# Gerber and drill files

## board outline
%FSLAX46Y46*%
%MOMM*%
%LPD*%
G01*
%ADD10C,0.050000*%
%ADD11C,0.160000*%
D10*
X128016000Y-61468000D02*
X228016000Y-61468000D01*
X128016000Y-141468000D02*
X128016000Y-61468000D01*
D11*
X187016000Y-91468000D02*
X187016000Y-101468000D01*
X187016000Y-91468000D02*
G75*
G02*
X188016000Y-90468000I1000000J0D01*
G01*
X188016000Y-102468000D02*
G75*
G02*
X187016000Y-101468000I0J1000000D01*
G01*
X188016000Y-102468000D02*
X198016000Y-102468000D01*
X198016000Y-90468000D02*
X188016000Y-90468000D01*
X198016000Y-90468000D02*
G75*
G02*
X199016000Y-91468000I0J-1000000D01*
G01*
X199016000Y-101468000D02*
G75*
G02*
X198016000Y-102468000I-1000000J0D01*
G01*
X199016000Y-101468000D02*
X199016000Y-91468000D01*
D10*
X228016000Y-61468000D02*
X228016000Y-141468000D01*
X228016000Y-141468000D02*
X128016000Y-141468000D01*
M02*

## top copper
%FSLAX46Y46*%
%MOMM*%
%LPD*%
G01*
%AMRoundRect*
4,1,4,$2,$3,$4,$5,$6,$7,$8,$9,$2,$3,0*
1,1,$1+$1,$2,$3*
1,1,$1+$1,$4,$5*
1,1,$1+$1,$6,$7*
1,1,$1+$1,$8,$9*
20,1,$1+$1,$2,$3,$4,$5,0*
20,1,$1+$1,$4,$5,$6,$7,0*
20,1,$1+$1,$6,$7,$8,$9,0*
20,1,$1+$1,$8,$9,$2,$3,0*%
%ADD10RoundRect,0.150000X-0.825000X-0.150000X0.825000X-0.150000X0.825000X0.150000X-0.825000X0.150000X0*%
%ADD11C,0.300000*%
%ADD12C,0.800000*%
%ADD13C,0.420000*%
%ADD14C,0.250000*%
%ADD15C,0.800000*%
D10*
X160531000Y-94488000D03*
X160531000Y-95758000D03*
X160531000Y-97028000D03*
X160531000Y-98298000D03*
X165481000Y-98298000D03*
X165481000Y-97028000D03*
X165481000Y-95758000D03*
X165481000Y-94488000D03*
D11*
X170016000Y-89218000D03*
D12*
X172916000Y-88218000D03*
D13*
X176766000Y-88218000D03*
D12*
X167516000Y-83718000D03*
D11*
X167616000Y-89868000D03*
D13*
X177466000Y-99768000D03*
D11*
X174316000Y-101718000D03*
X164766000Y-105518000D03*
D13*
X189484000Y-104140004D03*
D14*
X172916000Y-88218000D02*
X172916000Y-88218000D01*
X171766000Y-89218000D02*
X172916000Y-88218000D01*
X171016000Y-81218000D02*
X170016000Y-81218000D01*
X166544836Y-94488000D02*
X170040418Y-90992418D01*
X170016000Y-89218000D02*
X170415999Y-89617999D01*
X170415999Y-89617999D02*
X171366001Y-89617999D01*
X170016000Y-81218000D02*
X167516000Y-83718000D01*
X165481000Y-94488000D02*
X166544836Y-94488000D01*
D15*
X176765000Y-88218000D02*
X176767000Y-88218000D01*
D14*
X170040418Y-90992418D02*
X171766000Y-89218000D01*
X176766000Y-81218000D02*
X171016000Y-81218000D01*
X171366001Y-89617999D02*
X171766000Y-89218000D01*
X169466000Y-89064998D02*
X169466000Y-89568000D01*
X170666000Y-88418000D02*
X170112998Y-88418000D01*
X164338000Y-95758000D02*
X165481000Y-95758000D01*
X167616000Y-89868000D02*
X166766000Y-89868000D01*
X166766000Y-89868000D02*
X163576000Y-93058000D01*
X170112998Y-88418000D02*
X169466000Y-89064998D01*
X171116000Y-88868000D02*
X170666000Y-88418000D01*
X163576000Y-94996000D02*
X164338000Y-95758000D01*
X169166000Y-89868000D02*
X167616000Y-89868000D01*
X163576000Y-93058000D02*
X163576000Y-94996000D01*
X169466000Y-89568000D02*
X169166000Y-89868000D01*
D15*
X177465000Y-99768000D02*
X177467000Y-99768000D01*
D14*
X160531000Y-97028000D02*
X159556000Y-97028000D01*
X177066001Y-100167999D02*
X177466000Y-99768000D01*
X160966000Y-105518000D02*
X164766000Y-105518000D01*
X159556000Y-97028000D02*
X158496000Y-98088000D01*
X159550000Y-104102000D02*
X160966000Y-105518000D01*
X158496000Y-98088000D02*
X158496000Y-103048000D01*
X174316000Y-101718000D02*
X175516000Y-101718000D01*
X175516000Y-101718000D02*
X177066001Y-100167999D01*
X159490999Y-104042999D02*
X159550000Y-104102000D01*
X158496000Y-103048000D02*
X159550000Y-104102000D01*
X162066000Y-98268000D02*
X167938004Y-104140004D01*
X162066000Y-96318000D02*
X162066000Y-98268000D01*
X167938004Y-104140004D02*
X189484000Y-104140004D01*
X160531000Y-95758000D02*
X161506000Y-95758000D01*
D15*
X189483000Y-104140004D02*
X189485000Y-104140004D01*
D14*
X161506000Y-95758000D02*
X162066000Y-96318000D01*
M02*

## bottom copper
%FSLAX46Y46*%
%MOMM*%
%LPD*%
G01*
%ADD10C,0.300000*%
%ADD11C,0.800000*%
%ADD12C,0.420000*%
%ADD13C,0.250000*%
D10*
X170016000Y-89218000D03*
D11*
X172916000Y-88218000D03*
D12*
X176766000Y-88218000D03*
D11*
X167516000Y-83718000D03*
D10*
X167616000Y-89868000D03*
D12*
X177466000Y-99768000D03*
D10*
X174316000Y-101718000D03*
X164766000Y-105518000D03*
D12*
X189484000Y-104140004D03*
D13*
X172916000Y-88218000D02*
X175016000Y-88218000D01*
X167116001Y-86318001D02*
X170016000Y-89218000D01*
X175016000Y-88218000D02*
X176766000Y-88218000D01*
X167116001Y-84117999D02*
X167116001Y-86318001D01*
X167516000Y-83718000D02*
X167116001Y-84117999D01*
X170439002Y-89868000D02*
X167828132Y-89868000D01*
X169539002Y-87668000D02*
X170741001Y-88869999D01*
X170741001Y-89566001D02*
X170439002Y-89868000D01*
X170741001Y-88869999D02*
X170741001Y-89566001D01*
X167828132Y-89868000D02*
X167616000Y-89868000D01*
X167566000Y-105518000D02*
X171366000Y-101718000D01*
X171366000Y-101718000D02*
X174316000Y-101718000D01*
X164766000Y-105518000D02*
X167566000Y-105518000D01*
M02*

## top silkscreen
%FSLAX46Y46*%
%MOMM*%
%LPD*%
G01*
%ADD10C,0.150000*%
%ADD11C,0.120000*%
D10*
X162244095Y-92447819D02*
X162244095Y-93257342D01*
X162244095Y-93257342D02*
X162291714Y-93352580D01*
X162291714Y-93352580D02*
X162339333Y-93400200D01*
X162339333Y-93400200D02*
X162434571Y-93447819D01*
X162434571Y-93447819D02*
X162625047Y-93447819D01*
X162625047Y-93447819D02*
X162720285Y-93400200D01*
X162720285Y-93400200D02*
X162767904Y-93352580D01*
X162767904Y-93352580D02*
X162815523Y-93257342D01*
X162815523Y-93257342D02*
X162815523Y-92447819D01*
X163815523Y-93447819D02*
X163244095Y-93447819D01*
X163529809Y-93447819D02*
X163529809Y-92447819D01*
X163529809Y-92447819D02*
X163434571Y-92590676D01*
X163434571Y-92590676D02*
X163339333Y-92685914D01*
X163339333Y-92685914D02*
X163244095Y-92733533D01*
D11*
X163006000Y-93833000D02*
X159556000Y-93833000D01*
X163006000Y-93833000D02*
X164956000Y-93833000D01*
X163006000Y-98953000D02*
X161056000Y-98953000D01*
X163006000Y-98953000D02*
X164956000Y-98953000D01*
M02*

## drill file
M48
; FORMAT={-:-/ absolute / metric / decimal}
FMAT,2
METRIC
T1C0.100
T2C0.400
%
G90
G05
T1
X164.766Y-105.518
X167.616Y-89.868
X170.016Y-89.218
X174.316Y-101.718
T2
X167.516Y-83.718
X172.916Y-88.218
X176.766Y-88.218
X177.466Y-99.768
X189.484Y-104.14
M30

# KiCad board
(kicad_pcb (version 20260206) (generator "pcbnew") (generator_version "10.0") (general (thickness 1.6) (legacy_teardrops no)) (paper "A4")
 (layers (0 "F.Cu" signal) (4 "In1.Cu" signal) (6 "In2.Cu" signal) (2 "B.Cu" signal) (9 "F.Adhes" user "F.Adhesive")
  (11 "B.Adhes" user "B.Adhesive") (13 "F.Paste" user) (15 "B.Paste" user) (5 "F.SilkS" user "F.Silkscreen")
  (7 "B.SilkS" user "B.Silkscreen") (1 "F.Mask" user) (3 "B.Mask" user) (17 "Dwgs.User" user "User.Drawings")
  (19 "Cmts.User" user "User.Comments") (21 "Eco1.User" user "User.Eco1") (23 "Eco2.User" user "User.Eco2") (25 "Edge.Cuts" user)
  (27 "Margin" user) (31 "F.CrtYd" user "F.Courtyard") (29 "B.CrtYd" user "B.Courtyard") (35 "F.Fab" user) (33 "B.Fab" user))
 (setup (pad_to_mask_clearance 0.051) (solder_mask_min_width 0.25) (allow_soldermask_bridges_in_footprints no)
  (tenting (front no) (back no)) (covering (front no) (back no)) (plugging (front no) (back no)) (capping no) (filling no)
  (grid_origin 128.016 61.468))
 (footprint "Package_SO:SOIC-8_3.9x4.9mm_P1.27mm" (layer "F.Cu") (at 163.006 96.393)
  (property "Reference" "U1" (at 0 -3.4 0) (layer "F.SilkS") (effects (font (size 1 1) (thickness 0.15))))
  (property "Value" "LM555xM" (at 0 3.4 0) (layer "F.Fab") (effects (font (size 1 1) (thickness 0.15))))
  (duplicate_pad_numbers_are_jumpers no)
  (fp_line (start 0 -2.56) (end -3.45 -2.56) (stroke (width 0.12) (type solid)) (layer "F.SilkS"))
  (fp_line (start 0 -2.56) (end 1.95 -2.56) (stroke (width 0.12) (type solid)) (layer "F.SilkS"))
  (fp_line (start 0 2.56) (end -1.95 2.56) (stroke (width 0.12) (type solid)) (layer "F.SilkS"))
  (fp_line (start 0 2.56) (end 1.95 2.56) (stroke (width 0.12) (type solid)) (layer "F.SilkS"))
  (pad "1" smd roundrect (at -2.475 -1.905) (size 1.95 0.6) (layers "F.Cu" "F.Mask" "F.Paste") (roundrect_rratio 0.25) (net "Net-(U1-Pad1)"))
  (pad "2" smd roundrect (at -2.475 -0.635) (size 1.95 0.6) (layers "F.Cu" "F.Mask" "F.Paste") (roundrect_rratio 0.25) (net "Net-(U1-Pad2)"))
  (pad "3" smd roundrect (at -2.475 0.635) (size 1.95 0.6) (layers "F.Cu" "F.Mask" "F.Paste") (roundrect_rratio 0.25) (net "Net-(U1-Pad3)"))
  (pad "4" smd roundrect (at -2.475 1.905) (size 1.95 0.6) (layers "F.Cu" "F.Mask" "F.Paste") (roundrect_rratio 0.25) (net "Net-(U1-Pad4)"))
  (pad "5" smd roundrect (at 2.475 1.905) (size 1.95 0.6) (layers "F.Cu" "F.Mask" "F.Paste") (roundrect_rratio 0.25) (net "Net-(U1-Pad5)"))
  (pad "6" smd roundrect (at 2.475 0.635) (size 1.95 0.6) (layers "F.Cu" "F.Mask" "F.Paste") (roundrect_rratio 0.25) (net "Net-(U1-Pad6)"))
  (pad "7" smd roundrect (at 2.475 -0.635) (size 1.95 0.6) (layers "F.Cu" "F.Mask" "F.Paste") (roundrect_rratio 0.25) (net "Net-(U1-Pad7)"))
  (pad "8" smd roundrect (at 2.475 -1.905) (size 1.95 0.6) (layers "F.Cu" "F.Mask" "F.Paste") (roundrect_rratio 0.25) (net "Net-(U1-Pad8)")))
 (gr_line (start 128.016 61.468) (end 228.016 61.468) (stroke (width 0.05) (type solid)) (layer "Edge.Cuts"))
 (gr_line (start 128.016 141.468) (end 128.016 61.468) (stroke (width 0.05) (type solid)) (layer "Edge.Cuts"))
 (gr_line (start 187.016 91.468) (end 187.016 101.468) (stroke (width 0.16) (type solid)) (layer "Edge.Cuts"))
 (gr_arc (start 187.016 91.468) (mid 187.308893 90.760893) (end 188.016 90.468) (stroke (width 0.16) (type solid)) (layer "Edge.Cuts"))
 (gr_arc (start 188.016 102.468) (mid 187.308893 102.175107) (end 187.016 101.468) (stroke (width 0.16) (type solid)) (layer "Edge.Cuts"))
 (gr_line (start 188.016 102.468) (end 198.016 102.468) (stroke (width 0.16) (type solid)) (layer "Edge.Cuts"))
 (gr_line (start 198.016 90.468) (end 188.016 90.468) (stroke (width 0.16) (type solid)) (layer "Edge.Cuts"))
 (gr_arc (start 198.016 90.468) (mid 198.723107 90.760893) (end 199.016 91.468) (stroke (width 0.16) (type solid)) (layer "Edge.Cuts"))
 (gr_arc (start 199.016 101.468) (mid 198.723107 102.175107) (end 198.016 102.468) (stroke (width 0.16) (type solid)) (layer "Edge.Cuts"))
 (gr_line (start 199.016 101.468) (end 199.016 91.468) (stroke (width 0.16) (type solid)) (layer "Edge.Cuts"))
 (gr_line (start 228.016 61.468) (end 228.016 141.468) (stroke (width 0.05) (type solid)) (layer "Edge.Cuts"))
 (gr_line (start 228.016 141.468) (end 128.016 141.468) (stroke (width 0.05) (type solid)) (layer "Edge.Cuts"))
 (segment (start 172.916 88.218) (end 172.916 88.218) (width 0.25) (layer "F.Cu") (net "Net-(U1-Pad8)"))
 (segment (start 171.766 89.218) (end 172.916 88.218) (width 0.25) (layer "F.Cu") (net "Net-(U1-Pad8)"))
 (segment (start 171.016 81.218) (end 170.016 81.218) (width 0.25) (layer "F.Cu") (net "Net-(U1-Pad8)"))
 (segment (start 166.544836 94.488) (end 170.040418 90.992418) (width 0.25) (layer "F.Cu") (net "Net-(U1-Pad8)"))
 (segment (start 170.016 89.218) (end 170.415999 89.617999) (width 0.25) (layer "F.Cu") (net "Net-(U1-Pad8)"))
 (segment (start 170.415999 89.617999) (end 171.366001 89.617999) (width 0.25) (layer "F.Cu") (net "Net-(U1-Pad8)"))
 (segment (start 170.016 81.218) (end 167.516 83.718) (width 0.25) (layer "F.Cu") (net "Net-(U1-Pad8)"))
 (segment (start 165.481 94.488) (end 166.544836 94.488) (width 0.25) (layer "F.Cu") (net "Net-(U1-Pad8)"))
 (segment (start 176.765 88.218) (end 176.767 88.218) (width 0.8) (layer "F.Cu") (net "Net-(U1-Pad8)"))
 (segment (start 170.040418 90.992418) (end 171.766 89.218) (width 0.25) (layer "F.Cu") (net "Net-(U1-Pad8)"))
 (segment (start 176.766 81.218) (end 171.016 81.218) (width 0.25) (layer "F.Cu") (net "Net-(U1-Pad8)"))
 (segment (start 171.366001 89.617999) (end 171.766 89.218) (width 0.25) (layer "F.Cu") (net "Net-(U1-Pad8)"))
 (via (at 170.016 89.218) (size 0.3) (drill 0.1) (layers "F.Cu" "B.Cu") (capping no) (covering (front no) (back no))
  (plugging (front no) (back no)) (filling no) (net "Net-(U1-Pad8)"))
 (via (at 172.916 88.218) (size 0.8) (drill 0.4) (layers "F.Cu" "B.Cu") (capping no) (covering (front no) (back no))
  (plugging (front no) (back no)) (filling no) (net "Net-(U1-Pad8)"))
 (via (at 176.766 88.218) (size 0.42) (drill 0.4) (layers "F.Cu" "B.Cu") (capping no) (covering (front no) (back no))
  (plugging (front no) (back no)) (filling no) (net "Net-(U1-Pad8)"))
 (via (at 167.516 83.718) (size 0.8) (drill 0.4) (layers "F.Cu" "B.Cu") (capping no) (covering (front no) (back no))
  (plugging (front no) (back no)) (filling no) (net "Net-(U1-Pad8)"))
 (segment (start 172.916 88.218) (end 175.016 88.218) (width 0.25) (layer "B.Cu") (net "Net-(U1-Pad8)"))
 (segment (start 167.116001 86.318001) (end 170.016 89.218) (width 0.25) (layer "B.Cu") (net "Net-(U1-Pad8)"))
 (segment (start 175.016 88.218) (end 176.766 88.218) (width 0.25) (layer "B.Cu") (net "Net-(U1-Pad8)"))
 (segment (start 167.116001 84.117999) (end 167.116001 86.318001) (width 0.25) (layer "B.Cu") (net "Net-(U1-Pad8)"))
 (segment (start 167.516 83.718) (end 167.116001 84.117999) (width 0.25) (layer "B.Cu") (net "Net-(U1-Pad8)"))
 (segment (start 169.466 89.064998) (end 169.466 89.568) (width 0.25) (layer "F.Cu") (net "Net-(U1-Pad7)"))
 (segment (start 170.666 88.418) (end 170.112998 88.418) (width 0.25) (layer "F.Cu") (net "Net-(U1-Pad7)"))
 (segment (start 164.338 95.758) (end 165.481 95.758) (width 0.25) (layer "F.Cu") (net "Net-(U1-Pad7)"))
 (segment (start 167.616 89.868) (end 166.766 89.868) (width 0.25) (layer "F.Cu") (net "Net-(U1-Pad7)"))
 (segment (start 166.766 89.868) (end 163.576 93.058) (width 0.25) (layer "F.Cu") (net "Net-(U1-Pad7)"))
 (segment (start 170.112998 88.418) (end 169.466 89.064998) (width 0.25) (layer "F.Cu") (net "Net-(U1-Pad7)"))
 (segment (start 171.116 88.868) (end 170.666 88.418) (width 0.25) (layer "F.Cu") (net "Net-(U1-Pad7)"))
 (segment (start 163.576 94.996) (end 164.338 95.758) (width 0.25) (layer "F.Cu") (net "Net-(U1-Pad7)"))
 (segment (start 169.166 89.868) (end 167.616 89.868) (width 0.25) (layer "F.Cu") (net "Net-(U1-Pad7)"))
 (segment (start 163.576 93.058) (end 163.576 94.996) (width 0.25) (layer "F.Cu") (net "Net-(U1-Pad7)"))
 (segment (start 169.466 89.568) (end 169.166 89.868) (width 0.25) (layer "F.Cu") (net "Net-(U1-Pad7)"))
 (via (at 167.616 89.868) (size 0.3) (drill 0.1) (layers "F.Cu" "B.Cu") (capping no) (covering (front no) (back no))
  (plugging (front no) (back no)) (filling no) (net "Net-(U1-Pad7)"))
 (segment (start 170.439002 89.868) (end 167.828132 89.868) (width 0.25) (layer "B.Cu") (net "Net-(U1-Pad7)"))
 (segment (start 169.539002 87.668) (end 170.741001 88.869999) (width 0.25) (layer "B.Cu") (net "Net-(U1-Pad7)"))
 (segment (start 170.741001 89.566001) (end 170.439002 89.868) (width 0.25) (layer "B.Cu") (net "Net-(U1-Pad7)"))
 (segment (start 170.741001 88.869999) (end 170.741001 89.566001) (width 0.25) (layer "B.Cu") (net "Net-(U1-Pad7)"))
 (segment (start 167.828132 89.868) (end 167.616 89.868) (width 0.25) (layer "B.Cu") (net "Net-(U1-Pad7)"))
 (segment (start 177.465 99.768) (end 177.467 99.768) (width 0.8) (layer "F.Cu") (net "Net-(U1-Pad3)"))
 (segment (start 160.531 97.028) (end 159.556 97.028) (width 0.25) (layer "F.Cu") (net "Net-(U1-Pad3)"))
 (segment (start 177.066001 100.167999) (end 177.466 99.768) (width 0.25) (layer "F.Cu") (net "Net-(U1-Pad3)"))
 (segment (start 160.966 105.518) (end 164.766 105.518) (width 0.25) (layer "F.Cu") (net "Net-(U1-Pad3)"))
 (segment (start 159.556 97.028) (end 158.496 98.088) (width 0.25) (layer "F.Cu") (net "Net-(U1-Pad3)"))
 (segment (start 159.55 104.102) (end 160.966 105.518) (width 0.25) (layer "F.Cu") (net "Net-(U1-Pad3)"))
 (segment (start 158.496 98.088) (end 158.496 103.048) (width 0.25) (layer "F.Cu") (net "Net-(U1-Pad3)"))
 (segment (start 174.316 101.718) (end 175.516 101.718) (width 0.25) (layer "F.Cu") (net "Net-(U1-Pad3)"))
 (segment (start 175.516 101.718) (end 177.066001 100.167999) (width 0.25) (layer "F.Cu") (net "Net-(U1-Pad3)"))
 (segment (start 159.490999 104.042999) (end 159.55 104.102) (width 0.25) (layer "F.Cu") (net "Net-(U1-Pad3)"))
 (segment (start 158.496 103.048) (end 159.55 104.102) (width 0.25) (layer "F.Cu") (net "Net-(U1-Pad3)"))
 (via (at 177.466 99.768) (size 0.42) (drill 0.4) (layers "F.Cu" "B.Cu") (capping no) (covering (front no) (back no))
  (plugging (front no) (back no)) (filling no) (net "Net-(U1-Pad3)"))
 (via (at 174.316 101.718) (size 0.3) (drill 0.1) (layers "F.Cu" "B.Cu") (capping no) (covering (front no) (back no))
  (plugging (front no) (back no)) (filling no) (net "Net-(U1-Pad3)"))
 (via (at 164.766 105.518) (size 0.3) (drill 0.1) (layers "F.Cu" "B.Cu") (capping no) (covering (front no) (back no))
  (plugging (front no) (back no)) (filling no) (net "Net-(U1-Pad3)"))
 (segment (start 167.566 105.518) (end 171.366 101.718) (width 0.25) (layer "B.Cu") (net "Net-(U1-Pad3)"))
 (segment (start 171.366 101.718) (end 174.316 101.718) (width 0.25) (layer "B.Cu") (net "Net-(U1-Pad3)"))
 (segment (start 164.766 105.518) (end 167.566 105.518) (width 0.25) (layer "B.Cu") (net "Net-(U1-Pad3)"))
 (segment (start 162.066 98.268) (end 167.938004 104.140004) (width 0.25) (layer "F.Cu") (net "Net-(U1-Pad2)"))
 (segment (start 162.066 96.318) (end 162.066 98.268) (width 0.25) (layer "F.Cu") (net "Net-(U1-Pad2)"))
 (segment (start 167.938004 104.140004) (end 189.484 104.140004) (width 0.25) (layer "F.Cu") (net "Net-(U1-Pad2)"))
 (segment (start 160.531 95.758) (end 161.506 95.758) (width 0.25) (layer "F.Cu") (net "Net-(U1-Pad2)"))
 (segment (start 189.483 104.140004) (end 189.485 104.140004) (width 0.8) (layer "F.Cu") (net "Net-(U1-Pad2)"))
 (segment (start 161.506 95.758) (end 162.066 96.318) (width 0.25) (layer "F.Cu") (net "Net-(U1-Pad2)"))
 (via (at 189.484 104.140004) (size 0.42) (drill 0.4) (layers "F.Cu" "B.Cu") (capping no) (covering (front no) (back no))
  (plugging (front no) (back no)) (filling no) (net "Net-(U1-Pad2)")))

